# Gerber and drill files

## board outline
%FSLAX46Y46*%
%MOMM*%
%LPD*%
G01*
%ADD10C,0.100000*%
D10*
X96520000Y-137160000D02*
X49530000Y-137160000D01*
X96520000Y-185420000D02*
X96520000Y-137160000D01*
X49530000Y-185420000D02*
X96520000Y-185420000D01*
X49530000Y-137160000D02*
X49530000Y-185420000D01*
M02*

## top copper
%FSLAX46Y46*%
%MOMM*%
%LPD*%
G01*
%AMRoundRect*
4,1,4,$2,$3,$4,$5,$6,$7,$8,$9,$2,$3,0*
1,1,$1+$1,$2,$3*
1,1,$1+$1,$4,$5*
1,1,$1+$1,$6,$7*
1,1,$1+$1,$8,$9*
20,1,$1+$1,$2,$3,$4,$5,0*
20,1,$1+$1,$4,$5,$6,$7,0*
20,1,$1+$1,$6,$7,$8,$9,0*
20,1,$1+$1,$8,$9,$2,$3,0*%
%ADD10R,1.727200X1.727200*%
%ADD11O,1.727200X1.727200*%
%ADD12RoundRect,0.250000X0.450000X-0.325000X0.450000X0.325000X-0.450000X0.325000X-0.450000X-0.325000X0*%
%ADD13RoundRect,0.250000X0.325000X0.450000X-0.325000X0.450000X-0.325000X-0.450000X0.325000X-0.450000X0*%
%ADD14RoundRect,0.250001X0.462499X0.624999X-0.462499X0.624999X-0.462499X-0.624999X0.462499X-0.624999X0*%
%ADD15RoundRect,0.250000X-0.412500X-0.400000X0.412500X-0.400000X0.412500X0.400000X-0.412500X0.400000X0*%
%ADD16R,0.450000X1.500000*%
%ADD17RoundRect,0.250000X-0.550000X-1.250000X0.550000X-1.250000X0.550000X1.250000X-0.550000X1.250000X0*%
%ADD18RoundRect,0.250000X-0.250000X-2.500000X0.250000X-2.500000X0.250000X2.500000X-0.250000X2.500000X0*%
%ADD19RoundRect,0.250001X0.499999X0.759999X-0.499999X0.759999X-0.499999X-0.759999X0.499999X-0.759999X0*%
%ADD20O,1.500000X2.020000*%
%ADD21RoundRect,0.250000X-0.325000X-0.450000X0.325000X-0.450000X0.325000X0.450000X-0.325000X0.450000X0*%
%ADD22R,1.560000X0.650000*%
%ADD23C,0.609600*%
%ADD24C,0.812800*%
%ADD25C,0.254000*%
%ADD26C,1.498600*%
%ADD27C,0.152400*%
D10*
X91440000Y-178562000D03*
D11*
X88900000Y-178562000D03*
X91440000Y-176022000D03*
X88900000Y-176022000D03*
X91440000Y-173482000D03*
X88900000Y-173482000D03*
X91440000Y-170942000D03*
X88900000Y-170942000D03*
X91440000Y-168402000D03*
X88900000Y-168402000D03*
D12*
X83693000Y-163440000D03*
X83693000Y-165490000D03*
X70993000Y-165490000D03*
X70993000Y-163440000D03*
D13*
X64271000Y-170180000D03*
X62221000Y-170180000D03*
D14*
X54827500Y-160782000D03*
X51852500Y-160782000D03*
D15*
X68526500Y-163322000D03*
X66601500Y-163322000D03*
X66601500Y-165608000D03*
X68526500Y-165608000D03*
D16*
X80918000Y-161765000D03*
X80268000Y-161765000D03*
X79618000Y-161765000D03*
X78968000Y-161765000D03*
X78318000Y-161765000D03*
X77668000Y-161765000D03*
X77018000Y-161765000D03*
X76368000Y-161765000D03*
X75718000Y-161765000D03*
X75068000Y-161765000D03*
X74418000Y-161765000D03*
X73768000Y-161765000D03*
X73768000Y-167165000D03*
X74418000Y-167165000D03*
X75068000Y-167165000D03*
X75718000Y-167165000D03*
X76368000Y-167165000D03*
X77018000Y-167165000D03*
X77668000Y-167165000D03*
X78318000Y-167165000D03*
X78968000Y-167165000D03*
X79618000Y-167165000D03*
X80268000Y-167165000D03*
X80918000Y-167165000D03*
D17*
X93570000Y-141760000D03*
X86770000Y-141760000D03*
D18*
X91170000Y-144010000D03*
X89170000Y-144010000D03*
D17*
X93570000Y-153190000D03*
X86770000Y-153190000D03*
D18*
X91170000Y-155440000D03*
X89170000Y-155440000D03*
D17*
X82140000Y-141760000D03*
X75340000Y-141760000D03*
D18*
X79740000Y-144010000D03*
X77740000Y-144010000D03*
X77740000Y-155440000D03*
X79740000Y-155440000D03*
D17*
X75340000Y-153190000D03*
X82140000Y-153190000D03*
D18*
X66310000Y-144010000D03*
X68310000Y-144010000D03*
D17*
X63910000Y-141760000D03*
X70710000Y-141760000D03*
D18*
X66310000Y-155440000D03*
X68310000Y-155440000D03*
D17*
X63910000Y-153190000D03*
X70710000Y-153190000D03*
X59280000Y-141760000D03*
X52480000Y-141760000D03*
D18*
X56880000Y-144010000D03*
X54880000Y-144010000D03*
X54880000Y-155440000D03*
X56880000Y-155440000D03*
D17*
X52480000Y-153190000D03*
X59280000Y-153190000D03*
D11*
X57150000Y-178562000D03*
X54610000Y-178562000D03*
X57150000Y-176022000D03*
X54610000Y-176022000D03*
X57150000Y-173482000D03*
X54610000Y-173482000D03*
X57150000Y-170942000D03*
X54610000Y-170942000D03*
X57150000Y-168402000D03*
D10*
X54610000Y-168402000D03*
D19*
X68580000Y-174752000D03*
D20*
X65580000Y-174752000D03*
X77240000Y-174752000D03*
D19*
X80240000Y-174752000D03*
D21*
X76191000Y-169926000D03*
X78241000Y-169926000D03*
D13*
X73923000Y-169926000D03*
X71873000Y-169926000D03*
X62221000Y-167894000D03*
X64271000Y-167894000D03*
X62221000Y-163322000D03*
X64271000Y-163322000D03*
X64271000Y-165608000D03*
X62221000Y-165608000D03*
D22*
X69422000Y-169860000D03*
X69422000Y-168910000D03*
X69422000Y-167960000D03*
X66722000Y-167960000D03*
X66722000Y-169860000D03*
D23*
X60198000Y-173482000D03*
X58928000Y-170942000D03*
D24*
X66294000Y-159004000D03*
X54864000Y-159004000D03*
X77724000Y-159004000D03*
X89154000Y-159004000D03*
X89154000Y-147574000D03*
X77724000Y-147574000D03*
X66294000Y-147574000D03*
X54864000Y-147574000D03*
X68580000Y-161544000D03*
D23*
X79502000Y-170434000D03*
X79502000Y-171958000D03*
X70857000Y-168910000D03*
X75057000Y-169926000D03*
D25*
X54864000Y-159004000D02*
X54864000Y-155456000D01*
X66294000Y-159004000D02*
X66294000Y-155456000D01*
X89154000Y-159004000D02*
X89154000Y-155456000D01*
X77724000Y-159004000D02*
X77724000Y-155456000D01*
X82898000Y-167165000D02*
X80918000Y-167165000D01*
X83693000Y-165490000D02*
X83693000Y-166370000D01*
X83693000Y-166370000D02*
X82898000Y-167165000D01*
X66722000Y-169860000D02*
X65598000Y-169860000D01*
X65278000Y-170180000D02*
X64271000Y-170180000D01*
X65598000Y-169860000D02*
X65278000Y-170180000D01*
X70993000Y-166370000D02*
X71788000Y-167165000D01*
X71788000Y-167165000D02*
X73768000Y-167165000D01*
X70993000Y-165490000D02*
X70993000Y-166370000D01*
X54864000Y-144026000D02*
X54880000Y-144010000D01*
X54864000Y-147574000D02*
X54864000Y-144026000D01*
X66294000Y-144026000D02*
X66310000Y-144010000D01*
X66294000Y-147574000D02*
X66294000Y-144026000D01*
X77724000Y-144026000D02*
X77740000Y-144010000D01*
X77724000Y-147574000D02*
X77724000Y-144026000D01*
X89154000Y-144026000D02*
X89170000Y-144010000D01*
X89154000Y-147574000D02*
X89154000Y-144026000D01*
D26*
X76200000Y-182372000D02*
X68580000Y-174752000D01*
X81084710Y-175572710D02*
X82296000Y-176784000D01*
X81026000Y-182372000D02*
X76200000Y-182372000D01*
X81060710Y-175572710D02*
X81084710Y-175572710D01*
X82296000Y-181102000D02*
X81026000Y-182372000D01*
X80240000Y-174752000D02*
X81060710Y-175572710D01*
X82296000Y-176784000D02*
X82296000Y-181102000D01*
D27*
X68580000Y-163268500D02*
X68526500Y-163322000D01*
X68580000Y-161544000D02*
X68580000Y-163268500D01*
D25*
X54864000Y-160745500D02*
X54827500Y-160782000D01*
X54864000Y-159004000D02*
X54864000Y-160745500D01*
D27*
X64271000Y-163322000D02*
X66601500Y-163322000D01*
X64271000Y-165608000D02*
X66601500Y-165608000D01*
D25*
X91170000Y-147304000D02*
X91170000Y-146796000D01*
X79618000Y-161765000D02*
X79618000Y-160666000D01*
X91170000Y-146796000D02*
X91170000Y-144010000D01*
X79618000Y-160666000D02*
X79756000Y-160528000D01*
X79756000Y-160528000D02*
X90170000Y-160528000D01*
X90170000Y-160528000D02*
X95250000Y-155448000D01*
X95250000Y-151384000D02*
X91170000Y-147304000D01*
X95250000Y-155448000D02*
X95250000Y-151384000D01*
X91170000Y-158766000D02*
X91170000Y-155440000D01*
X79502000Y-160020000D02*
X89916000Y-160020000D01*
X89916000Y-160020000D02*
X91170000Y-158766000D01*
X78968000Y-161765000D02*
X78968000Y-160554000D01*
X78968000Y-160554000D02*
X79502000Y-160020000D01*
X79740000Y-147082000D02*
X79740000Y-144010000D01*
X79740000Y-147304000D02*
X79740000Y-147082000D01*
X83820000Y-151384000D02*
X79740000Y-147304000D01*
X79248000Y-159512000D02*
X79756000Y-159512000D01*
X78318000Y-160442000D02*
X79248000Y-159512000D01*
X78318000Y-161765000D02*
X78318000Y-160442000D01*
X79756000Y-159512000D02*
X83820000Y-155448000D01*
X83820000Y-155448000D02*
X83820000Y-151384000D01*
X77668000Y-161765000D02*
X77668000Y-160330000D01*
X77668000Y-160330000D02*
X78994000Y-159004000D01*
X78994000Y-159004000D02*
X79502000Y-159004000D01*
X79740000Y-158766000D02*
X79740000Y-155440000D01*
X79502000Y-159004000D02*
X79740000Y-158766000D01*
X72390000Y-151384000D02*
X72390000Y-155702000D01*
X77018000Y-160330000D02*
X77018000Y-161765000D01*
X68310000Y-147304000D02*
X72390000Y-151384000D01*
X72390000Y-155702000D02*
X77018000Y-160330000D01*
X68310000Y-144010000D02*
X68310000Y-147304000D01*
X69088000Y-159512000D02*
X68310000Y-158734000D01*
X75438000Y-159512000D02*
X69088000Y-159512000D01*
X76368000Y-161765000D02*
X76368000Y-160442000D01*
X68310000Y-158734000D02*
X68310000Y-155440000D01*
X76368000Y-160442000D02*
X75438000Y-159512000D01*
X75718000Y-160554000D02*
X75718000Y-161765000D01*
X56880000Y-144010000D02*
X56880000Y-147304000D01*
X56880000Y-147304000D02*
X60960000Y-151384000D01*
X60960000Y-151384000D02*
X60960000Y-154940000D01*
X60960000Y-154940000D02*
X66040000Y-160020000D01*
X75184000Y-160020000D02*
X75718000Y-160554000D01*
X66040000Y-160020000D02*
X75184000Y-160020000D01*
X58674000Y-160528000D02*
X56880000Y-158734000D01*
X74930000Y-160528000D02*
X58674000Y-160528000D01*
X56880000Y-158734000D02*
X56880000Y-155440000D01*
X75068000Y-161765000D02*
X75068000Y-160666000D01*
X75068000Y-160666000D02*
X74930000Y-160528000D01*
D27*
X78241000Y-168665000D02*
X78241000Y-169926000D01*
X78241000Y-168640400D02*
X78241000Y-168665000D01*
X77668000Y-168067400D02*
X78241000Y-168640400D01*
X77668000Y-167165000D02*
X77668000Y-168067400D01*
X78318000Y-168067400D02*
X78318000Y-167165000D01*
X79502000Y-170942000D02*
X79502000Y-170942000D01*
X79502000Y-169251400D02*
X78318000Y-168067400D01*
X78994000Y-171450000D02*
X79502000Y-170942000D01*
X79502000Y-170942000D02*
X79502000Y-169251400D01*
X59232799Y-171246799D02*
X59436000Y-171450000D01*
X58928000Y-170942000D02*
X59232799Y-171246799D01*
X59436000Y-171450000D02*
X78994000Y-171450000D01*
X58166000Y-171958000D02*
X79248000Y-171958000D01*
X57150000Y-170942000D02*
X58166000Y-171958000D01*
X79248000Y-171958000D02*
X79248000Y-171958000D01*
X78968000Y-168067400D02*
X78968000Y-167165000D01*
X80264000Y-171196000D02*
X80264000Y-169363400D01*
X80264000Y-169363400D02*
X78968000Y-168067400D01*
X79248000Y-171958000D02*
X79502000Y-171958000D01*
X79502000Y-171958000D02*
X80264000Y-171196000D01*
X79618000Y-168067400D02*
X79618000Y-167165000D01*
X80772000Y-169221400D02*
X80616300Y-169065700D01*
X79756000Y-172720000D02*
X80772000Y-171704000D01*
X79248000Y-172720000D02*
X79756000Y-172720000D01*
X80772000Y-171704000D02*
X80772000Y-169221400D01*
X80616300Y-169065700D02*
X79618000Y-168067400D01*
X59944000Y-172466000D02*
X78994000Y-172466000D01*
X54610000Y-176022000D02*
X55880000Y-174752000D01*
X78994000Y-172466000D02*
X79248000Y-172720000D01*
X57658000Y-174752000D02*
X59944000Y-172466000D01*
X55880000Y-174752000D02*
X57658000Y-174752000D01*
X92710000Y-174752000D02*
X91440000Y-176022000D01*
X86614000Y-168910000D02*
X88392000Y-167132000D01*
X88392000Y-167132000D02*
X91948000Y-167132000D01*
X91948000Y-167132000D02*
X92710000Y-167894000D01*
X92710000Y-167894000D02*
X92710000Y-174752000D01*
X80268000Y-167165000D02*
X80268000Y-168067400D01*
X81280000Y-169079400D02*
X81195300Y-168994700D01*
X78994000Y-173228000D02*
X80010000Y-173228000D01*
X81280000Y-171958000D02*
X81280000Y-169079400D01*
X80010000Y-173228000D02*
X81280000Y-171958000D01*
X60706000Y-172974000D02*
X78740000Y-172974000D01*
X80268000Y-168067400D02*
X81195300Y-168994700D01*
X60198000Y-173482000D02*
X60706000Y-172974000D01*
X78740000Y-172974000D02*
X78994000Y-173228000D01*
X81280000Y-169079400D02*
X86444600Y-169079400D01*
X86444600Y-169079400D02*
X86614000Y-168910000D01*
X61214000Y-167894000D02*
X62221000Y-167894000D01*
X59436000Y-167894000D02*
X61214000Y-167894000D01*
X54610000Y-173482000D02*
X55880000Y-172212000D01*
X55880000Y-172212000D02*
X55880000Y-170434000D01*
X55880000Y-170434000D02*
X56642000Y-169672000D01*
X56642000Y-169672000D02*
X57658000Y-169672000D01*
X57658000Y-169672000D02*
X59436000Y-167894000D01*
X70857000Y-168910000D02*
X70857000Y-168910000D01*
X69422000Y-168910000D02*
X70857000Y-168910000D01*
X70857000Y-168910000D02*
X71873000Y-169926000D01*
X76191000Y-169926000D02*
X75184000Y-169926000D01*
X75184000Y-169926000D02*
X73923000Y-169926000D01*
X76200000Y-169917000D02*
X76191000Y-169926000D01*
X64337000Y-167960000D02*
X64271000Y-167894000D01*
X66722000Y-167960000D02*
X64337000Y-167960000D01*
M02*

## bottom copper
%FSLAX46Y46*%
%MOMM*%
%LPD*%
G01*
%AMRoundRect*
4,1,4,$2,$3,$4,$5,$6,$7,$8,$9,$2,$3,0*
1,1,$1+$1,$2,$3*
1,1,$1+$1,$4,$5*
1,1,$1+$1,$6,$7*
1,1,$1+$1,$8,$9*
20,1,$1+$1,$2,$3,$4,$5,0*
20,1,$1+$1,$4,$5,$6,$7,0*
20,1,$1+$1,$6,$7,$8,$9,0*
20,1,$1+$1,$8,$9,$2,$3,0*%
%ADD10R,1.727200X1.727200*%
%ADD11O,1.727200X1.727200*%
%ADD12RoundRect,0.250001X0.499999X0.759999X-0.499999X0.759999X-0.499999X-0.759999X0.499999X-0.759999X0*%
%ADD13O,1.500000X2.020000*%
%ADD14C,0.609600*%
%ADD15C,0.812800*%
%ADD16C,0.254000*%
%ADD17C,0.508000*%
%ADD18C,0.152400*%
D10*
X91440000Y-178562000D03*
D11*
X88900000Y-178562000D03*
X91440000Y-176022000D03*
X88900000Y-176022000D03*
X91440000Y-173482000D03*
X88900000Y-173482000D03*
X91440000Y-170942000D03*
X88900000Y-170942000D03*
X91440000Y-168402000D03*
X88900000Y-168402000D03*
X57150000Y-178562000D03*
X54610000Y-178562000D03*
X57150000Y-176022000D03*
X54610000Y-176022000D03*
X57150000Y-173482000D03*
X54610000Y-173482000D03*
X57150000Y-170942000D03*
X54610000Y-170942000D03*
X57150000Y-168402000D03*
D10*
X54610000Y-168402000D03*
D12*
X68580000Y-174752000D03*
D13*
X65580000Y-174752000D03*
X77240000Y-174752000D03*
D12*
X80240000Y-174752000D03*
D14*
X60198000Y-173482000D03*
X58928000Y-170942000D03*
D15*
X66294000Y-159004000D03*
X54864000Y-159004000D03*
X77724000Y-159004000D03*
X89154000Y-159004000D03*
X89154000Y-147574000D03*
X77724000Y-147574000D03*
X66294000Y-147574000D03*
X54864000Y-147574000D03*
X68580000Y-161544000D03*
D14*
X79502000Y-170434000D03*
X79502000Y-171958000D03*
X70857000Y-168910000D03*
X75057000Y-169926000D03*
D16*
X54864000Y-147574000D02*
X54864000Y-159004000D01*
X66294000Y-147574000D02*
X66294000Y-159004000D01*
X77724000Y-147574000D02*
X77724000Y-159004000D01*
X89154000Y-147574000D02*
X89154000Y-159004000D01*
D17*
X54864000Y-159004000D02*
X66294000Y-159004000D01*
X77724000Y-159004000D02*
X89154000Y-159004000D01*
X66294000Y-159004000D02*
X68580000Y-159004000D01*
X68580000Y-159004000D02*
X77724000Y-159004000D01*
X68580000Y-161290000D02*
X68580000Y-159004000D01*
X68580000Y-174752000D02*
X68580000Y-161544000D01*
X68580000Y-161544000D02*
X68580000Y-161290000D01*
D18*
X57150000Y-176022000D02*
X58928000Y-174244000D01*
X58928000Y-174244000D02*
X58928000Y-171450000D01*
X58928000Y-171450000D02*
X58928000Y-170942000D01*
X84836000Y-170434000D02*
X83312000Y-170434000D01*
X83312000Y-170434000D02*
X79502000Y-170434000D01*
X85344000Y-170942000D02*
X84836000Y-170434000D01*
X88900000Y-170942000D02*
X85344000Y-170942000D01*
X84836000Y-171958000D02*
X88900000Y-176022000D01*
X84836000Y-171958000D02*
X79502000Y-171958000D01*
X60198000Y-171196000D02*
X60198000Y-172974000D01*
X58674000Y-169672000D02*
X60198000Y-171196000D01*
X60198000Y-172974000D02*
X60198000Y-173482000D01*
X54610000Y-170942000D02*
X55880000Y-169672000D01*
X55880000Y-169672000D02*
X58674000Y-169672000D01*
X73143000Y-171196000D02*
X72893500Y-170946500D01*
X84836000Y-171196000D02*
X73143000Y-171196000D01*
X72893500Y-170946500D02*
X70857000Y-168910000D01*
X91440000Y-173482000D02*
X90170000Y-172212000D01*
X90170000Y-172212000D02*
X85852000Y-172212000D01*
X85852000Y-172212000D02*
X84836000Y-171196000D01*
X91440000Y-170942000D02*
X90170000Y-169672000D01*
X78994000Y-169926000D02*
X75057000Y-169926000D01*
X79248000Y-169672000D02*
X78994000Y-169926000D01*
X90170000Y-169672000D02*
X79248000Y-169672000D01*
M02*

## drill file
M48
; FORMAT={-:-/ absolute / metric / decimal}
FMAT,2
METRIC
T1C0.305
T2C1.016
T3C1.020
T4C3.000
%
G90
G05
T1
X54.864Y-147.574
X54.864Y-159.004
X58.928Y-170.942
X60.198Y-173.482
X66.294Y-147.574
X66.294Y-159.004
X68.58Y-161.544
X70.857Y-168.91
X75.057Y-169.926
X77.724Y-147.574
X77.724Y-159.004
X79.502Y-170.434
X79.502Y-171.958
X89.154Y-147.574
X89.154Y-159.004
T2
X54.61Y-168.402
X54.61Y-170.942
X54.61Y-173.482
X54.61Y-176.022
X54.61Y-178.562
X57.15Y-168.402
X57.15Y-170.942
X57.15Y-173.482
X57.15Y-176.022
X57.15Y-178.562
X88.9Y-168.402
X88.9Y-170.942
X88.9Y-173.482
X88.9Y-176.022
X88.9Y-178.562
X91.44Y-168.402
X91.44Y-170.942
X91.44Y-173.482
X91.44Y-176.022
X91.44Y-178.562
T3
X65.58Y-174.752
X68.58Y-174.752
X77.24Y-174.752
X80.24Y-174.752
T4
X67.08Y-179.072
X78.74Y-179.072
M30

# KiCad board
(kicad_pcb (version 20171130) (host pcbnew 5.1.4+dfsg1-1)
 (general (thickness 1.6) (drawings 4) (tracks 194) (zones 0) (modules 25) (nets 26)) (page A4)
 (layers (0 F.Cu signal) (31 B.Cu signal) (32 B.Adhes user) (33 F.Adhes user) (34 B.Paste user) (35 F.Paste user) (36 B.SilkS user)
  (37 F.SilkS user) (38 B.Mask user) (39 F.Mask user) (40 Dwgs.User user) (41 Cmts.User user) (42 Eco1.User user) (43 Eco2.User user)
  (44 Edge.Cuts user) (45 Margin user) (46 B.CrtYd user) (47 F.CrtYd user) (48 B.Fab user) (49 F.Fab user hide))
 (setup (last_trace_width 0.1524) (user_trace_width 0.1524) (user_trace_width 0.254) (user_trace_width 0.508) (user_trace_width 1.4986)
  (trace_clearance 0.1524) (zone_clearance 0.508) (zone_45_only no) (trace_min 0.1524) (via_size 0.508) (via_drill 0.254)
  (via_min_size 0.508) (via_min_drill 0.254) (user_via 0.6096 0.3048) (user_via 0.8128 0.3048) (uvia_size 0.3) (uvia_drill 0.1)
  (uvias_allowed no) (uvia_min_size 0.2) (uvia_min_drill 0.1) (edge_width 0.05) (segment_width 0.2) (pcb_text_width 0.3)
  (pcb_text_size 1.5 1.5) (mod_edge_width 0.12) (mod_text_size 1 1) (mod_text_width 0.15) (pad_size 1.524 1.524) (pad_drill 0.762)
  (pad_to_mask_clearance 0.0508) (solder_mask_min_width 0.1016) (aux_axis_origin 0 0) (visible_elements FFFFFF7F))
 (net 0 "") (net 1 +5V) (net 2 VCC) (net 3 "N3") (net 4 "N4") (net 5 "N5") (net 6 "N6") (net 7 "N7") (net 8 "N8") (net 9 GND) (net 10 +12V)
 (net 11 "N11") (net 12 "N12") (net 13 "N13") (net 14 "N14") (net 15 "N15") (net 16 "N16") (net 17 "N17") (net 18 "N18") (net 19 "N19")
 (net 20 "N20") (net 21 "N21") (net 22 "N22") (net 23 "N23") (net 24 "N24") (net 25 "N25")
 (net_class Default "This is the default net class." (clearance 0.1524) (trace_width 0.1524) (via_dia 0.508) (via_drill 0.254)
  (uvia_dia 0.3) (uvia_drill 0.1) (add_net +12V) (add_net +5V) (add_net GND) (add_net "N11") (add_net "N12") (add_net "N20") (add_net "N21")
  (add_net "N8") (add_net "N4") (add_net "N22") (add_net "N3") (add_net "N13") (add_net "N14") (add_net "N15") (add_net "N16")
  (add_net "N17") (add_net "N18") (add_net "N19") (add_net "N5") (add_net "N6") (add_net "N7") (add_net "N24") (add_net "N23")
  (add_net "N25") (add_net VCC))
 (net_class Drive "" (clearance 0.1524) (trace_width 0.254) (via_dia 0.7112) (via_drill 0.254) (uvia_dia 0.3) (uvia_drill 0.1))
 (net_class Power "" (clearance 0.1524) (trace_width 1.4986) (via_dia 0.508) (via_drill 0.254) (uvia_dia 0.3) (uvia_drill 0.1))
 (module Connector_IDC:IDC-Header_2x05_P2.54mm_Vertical (layer F.Cu) (at 91.44 178.562 180)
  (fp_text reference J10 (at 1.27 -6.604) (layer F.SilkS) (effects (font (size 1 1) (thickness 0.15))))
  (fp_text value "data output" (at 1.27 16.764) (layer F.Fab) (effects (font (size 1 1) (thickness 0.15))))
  (pad 1 thru_hole rect (at 0 0 180) (size 1.7272 1.7272) (drill 1.016) (layers *.Cu *.Mask) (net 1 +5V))
  (pad 2 thru_hole oval (at 2.54 0 180) (size 1.7272 1.7272) (drill 1.016) (layers *.Cu *.Mask) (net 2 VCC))
  (pad 3 thru_hole oval (at 0 2.54 180) (size 1.7272 1.7272) (drill 1.016) (layers *.Cu *.Mask) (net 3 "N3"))
  (pad 4 thru_hole oval (at 2.54 2.54 180) (size 1.7272 1.7272) (drill 1.016) (layers *.Cu *.Mask) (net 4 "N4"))
  (pad 5 thru_hole oval (at 0 5.08 180) (size 1.7272 1.7272) (drill 1.016) (layers *.Cu *.Mask) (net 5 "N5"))
  (pad 6 thru_hole oval (at 2.54 5.08 180) (size 1.7272 1.7272) (drill 1.016) (layers *.Cu *.Mask) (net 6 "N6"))
  (pad 7 thru_hole oval (at 0 7.62 180) (size 1.7272 1.7272) (drill 1.016) (layers *.Cu *.Mask) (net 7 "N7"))
  (pad 8 thru_hole oval (at 2.54 7.62 180) (size 1.7272 1.7272) (drill 1.016) (layers *.Cu *.Mask) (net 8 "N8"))
  (pad 9 thru_hole oval (at 0 10.16 180) (size 1.7272 1.7272) (drill 1.016) (layers *.Cu *.Mask) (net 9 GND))
  (pad 10 thru_hole oval (at 2.54 10.16 180) (size 1.7272 1.7272) (drill 1.016) (layers *.Cu *.Mask) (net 9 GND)))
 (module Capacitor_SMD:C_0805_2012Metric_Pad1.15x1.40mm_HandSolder (layer F.Cu) (at 83.693 164.465 90)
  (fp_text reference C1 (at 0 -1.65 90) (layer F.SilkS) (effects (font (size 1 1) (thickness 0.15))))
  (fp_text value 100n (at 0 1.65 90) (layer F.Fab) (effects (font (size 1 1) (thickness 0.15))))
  (pad 2 smd roundrect (at 1.025 0 90) (size 1.15 1.4) (layers F.Cu F.Paste F.Mask) (roundrect_rratio 0.217391) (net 9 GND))
  (pad 1 smd roundrect (at -1.025 0 90) (size 1.15 1.4) (layers F.Cu F.Paste F.Mask) (roundrect_rratio 0.217391) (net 1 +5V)))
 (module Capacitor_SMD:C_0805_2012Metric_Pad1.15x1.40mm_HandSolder (layer F.Cu) (at 70.993 164.465 90)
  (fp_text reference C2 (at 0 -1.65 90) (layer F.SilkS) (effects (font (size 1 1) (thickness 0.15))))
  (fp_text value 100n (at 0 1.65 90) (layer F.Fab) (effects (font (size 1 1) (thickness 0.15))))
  (pad 1 smd roundrect (at -1.025 0 90) (size 1.15 1.4) (layers F.Cu F.Paste F.Mask) (roundrect_rratio 0.217391) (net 2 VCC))
  (pad 2 smd roundrect (at 1.025 0 90) (size 1.15 1.4) (layers F.Cu F.Paste F.Mask) (roundrect_rratio 0.217391) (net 9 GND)))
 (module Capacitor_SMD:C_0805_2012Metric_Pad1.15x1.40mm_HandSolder (layer F.Cu) (at 63.246 170.18 180)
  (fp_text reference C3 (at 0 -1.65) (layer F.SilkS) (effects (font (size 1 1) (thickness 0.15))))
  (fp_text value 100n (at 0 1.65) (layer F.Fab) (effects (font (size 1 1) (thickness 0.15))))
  (pad 1 smd roundrect (at -1.025 0 180) (size 1.15 1.4) (layers F.Cu F.Paste F.Mask) (roundrect_rratio 0.217391) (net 2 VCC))
  (pad 2 smd roundrect (at 1.025 0 180) (size 1.15 1.4) (layers F.Cu F.Paste F.Mask) (roundrect_rratio 0.217391) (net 9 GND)))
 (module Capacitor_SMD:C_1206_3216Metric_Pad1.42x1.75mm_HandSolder (layer F.Cu) (at 53.34 160.782 180)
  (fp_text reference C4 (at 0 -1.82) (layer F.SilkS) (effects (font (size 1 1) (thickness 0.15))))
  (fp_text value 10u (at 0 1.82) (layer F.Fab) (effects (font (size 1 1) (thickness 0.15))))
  (pad 1 smd roundrect (at -1.4875 0 180) (size 1.425 1.75) (layers F.Cu F.Paste F.Mask) (roundrect_rratio 0.175439) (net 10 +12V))
  (pad 2 smd roundrect (at 1.4875 0 180) (size 1.425 1.75) (layers F.Cu F.Paste F.Mask) (roundrect_rratio 0.175439) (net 9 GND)))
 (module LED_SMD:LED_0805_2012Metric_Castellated (layer F.Cu) (at 67.564 163.322)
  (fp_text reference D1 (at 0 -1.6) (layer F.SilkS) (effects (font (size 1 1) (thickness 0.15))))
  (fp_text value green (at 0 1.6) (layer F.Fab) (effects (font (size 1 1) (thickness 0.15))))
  (pad 2 smd roundrect (at 0.9625 0) (size 1.325 1.3) (layers F.Cu F.Paste F.Mask) (roundrect_rratio 0.192308) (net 10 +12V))
  (pad 1 smd roundrect (at -0.9625 0) (size 1.325 1.3) (layers F.Cu F.Paste F.Mask) (roundrect_rratio 0.192308) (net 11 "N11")))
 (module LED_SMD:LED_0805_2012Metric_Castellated (layer F.Cu) (at 67.564 165.608)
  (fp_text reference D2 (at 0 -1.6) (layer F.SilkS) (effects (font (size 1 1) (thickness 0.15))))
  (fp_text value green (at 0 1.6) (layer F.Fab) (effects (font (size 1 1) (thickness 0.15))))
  (pad 1 smd roundrect (at -0.9625 0) (size 1.325 1.3) (layers F.Cu F.Paste F.Mask) (roundrect_rratio 0.192308) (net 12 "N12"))
  (pad 2 smd roundrect (at 0.9625 0) (size 1.325 1.3) (layers F.Cu F.Paste F.Mask) (roundrect_rratio 0.192308) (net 1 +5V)))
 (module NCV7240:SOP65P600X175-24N (layer F.Cu) (at 77.343 164.465 270)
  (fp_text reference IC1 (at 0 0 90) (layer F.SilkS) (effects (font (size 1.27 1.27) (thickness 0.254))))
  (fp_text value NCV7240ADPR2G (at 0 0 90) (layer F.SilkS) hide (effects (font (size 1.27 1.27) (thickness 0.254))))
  (pad 1 smd rect (at -2.7 -3.575) (size 0.45 1.5) (layers F.Cu F.Paste F.Mask) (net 9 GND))
  (pad 2 smd rect (at -2.7 -2.925) (size 0.45 1.5) (layers F.Cu F.Paste F.Mask) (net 9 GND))
  (pad 3 smd rect (at -2.7 -2.275) (size 0.45 1.5) (layers F.Cu F.Paste F.Mask) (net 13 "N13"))
  (pad 4 smd rect (at -2.7 -1.625) (size 0.45 1.5) (layers F.Cu F.Paste F.Mask) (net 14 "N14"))
  (pad 5 smd rect (at -2.7 -0.975) (size 0.45 1.5) (layers F.Cu F.Paste F.Mask) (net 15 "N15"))
  (pad 6 smd rect (at -2.7 -0.325) (size 0.45 1.5) (layers F.Cu F.Paste F.Mask) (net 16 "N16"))
  (pad 7 smd rect (at -2.7 0.325) (size 0.45 1.5) (layers F.Cu F.Paste F.Mask) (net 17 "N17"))
  (pad 8 smd rect (at -2.7 0.975) (size 0.45 1.5) (layers F.Cu F.Paste F.Mask) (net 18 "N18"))
  (pad 9 smd rect (at -2.7 1.625) (size 0.45 1.5) (layers F.Cu F.Paste F.Mask) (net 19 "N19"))
  (pad 10 smd rect (at -2.7 2.275) (size 0.45 1.5) (layers F.Cu F.Paste F.Mask) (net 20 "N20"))
  (pad 11 smd rect (at -2.7 2.925) (size 0.45 1.5) (layers F.Cu F.Paste F.Mask) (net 9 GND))
  (pad 12 smd rect (at -2.7 3.575) (size 0.45 1.5) (layers F.Cu F.Paste F.Mask) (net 9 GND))
  (pad 13 smd rect (at 2.7 3.575) (size 0.45 1.5) (layers F.Cu F.Paste F.Mask) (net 2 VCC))
  (pad 14 smd rect (at 2.7 2.925) (size 0.45 1.5) (layers F.Cu F.Paste F.Mask) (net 9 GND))
  (pad 15 smd rect (at 2.7 2.275) (size 0.45 1.5) (layers F.Cu F.Paste F.Mask) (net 9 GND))
  (pad 16 smd rect (at 2.7 1.625) (size 0.45 1.5) (layers F.Cu F.Paste F.Mask) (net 9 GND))
  (pad 17 smd rect (at 2.7 0.975) (size 0.45 1.5) (layers F.Cu F.Paste F.Mask) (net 9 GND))
  (pad 18 smd rect (at 2.7 0.325) (size 0.45 1.5) (layers F.Cu F.Paste F.Mask) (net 9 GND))
  (pad 19 smd rect (at 2.7 -0.325) (size 0.45 1.5) (layers F.Cu F.Paste F.Mask) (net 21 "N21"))
  (pad 20 smd rect (at 2.7 -0.975) (size 0.45 1.5) (layers F.Cu F.Paste F.Mask) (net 8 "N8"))
  (pad 21 smd rect (at 2.7 -1.625) (size 0.45 1.5) (layers F.Cu F.Paste F.Mask) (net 4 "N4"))
  (pad 22 smd rect (at 2.7 -2.275) (size 0.45 1.5) (layers F.Cu F.Paste F.Mask) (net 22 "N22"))
  (pad 23 smd rect (at 2.7 -2.925) (size 0.45 1.5) (layers F.Cu F.Paste F.Mask) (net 3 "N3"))
  (pad 24 smd rect (at 2.7 -3.575) (size 0.45 1.5) (layers F.Cu F.Paste F.Mask) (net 1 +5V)))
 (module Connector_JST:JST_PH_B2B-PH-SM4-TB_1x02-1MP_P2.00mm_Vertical (layer F.Cu) (at 90.17 143.51)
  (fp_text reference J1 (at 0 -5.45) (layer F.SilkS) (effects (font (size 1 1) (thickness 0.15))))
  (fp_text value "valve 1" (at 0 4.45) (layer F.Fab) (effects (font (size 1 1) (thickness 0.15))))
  (pad MP smd roundrect (at 3.4 -1.75) (size 1.6 3) (layers F.Cu F.Paste F.Mask) (roundrect_rratio 0.15625))
  (pad MP smd roundrect (at -3.4 -1.75) (size 1.6 3) (layers F.Cu F.Paste F.Mask) (roundrect_rratio 0.15625))
  (pad 2 smd roundrect (at 1 0.5) (size 1 5.5) (layers F.Cu F.Paste F.Mask) (roundrect_rratio 0.25) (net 13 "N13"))
  (pad 1 smd roundrect (at -1 0.5) (size 1 5.5) (layers F.Cu F.Paste F.Mask) (roundrect_rratio 0.25) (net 10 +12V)))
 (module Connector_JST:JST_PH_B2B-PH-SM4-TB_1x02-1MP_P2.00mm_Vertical (layer F.Cu) (at 90.17 154.94)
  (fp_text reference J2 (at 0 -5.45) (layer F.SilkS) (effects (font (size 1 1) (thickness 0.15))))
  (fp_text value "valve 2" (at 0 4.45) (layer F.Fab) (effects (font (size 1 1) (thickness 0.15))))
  (pad MP smd roundrect (at 3.4 -1.75) (size 1.6 3) (layers F.Cu F.Paste F.Mask) (roundrect_rratio 0.15625))
  (pad MP smd roundrect (at -3.4 -1.75) (size 1.6 3) (layers F.Cu F.Paste F.Mask) (roundrect_rratio 0.15625))
  (pad 2 smd roundrect (at 1 0.5) (size 1 5.5) (layers F.Cu F.Paste F.Mask) (roundrect_rratio 0.25) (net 14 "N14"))
  (pad 1 smd roundrect (at -1 0.5) (size 1 5.5) (layers F.Cu F.Paste F.Mask) (roundrect_rratio 0.25) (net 10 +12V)))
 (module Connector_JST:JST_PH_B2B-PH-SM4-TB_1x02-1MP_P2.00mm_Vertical (layer F.Cu) (at 78.74 143.51)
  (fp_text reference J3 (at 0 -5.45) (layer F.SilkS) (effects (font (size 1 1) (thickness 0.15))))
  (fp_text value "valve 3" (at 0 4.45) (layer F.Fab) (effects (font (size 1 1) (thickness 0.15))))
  (pad MP smd roundrect (at 3.4 -1.75) (size 1.6 3) (layers F.Cu F.Paste F.Mask) (roundrect_rratio 0.15625))
  (pad MP smd roundrect (at -3.4 -1.75) (size 1.6 3) (layers F.Cu F.Paste F.Mask) (roundrect_rratio 0.15625))
  (pad 2 smd roundrect (at 1 0.5) (size 1 5.5) (layers F.Cu F.Paste F.Mask) (roundrect_rratio 0.25) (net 15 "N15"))
  (pad 1 smd roundrect (at -1 0.5) (size 1 5.5) (layers F.Cu F.Paste F.Mask) (roundrect_rratio 0.25) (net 10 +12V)))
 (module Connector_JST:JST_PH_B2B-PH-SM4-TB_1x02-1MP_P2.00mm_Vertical (layer F.Cu) (at 78.74 154.94)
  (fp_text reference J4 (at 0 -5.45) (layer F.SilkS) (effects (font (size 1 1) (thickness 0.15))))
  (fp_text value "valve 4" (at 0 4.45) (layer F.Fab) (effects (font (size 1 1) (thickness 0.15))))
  (pad 1 smd roundrect (at -1 0.5) (size 1 5.5) (layers F.Cu F.Paste F.Mask) (roundrect_rratio 0.25) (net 10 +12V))
  (pad 2 smd roundrect (at 1 0.5) (size 1 5.5) (layers F.Cu F.Paste F.Mask) (roundrect_rratio 0.25) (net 16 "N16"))
  (pad MP smd roundrect (at -3.4 -1.75) (size 1.6 3) (layers F.Cu F.Paste F.Mask) (roundrect_rratio 0.15625))
  (pad MP smd roundrect (at 3.4 -1.75) (size 1.6 3) (layers F.Cu F.Paste F.Mask) (roundrect_rratio 0.15625)))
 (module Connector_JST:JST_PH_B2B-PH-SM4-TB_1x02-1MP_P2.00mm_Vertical (layer F.Cu) (at 67.31 143.51)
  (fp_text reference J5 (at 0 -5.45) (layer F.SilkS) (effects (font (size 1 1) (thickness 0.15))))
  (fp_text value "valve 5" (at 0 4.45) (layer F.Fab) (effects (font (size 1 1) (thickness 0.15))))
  (pad 1 smd roundrect (at -1 0.5) (size 1 5.5) (layers F.Cu F.Paste F.Mask) (roundrect_rratio 0.25) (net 10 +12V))
  (pad 2 smd roundrect (at 1 0.5) (size 1 5.5) (layers F.Cu F.Paste F.Mask) (roundrect_rratio 0.25) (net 17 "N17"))
  (pad MP smd roundrect (at -3.4 -1.75) (size 1.6 3) (layers F.Cu F.Paste F.Mask) (roundrect_rratio 0.15625))
  (pad MP smd roundrect (at 3.4 -1.75) (size 1.6 3) (layers F.Cu F.Paste F.Mask) (roundrect_rratio 0.15625)))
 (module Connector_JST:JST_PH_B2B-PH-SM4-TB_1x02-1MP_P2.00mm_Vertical (layer F.Cu) (at 67.31 154.94)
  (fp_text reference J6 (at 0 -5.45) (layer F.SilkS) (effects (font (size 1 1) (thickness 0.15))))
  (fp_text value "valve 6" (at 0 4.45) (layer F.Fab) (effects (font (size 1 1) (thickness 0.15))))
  (pad 1 smd roundrect (at -1 0.5) (size 1 5.5) (layers F.Cu F.Paste F.Mask) (roundrect_rratio 0.25) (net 10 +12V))
  (pad 2 smd roundrect (at 1 0.5) (size 1 5.5) (layers F.Cu F.Paste F.Mask) (roundrect_rratio 0.25) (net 18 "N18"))
  (pad MP smd roundrect (at -3.4 -1.75) (size 1.6 3) (layers F.Cu F.Paste F.Mask) (roundrect_rratio 0.15625))
  (pad MP smd roundrect (at 3.4 -1.75) (size 1.6 3) (layers F.Cu F.Paste F.Mask) (roundrect_rratio 0.15625)))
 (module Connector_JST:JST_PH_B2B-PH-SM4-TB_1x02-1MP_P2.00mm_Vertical (layer F.Cu) (at 55.88 143.51)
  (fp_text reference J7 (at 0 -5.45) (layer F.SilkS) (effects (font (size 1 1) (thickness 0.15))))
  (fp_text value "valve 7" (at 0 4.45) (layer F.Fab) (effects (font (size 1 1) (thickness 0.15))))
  (pad MP smd roundrect (at 3.4 -1.75) (size 1.6 3) (layers F.Cu F.Paste F.Mask) (roundrect_rratio 0.15625))
  (pad MP smd roundrect (at -3.4 -1.75) (size 1.6 3) (layers F.Cu F.Paste F.Mask) (roundrect_rratio 0.15625))
  (pad 2 smd roundrect (at 1 0.5) (size 1 5.5) (layers F.Cu F.Paste F.Mask) (roundrect_rratio 0.25) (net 19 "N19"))
  (pad 1 smd roundrect (at -1 0.5) (size 1 5.5) (layers F.Cu F.Paste F.Mask) (roundrect_rratio 0.25) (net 10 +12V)))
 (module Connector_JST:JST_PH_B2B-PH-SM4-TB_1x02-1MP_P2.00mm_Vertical (layer F.Cu) (at 55.88 154.94)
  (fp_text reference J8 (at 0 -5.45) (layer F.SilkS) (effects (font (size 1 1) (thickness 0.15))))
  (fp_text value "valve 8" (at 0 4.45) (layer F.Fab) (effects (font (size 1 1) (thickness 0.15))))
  (pad 1 smd roundrect (at -1 0.5) (size 1 5.5) (layers F.Cu F.Paste F.Mask) (roundrect_rratio 0.25) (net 10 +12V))
  (pad 2 smd roundrect (at 1 0.5) (size 1 5.5) (layers F.Cu F.Paste F.Mask) (roundrect_rratio 0.25) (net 20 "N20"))
  (pad MP smd roundrect (at -3.4 -1.75) (size 1.6 3) (layers F.Cu F.Paste F.Mask) (roundrect_rratio 0.15625))
  (pad MP smd roundrect (at 3.4 -1.75) (size 1.6 3) (layers F.Cu F.Paste F.Mask) (roundrect_rratio 0.15625)))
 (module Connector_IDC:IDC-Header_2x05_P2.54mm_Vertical (layer F.Cu) (at 54.61 168.402)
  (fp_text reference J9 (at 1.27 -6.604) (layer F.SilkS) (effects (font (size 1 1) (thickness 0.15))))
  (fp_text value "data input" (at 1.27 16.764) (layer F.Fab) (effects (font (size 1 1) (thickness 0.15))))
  (pad 10 thru_hole oval (at 2.54 10.16) (size 1.7272 1.7272) (drill 1.016) (layers *.Cu *.Mask) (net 9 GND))
  (pad 9 thru_hole oval (at 0 10.16) (size 1.7272 1.7272) (drill 1.016) (layers *.Cu *.Mask) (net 9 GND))
  (pad 8 thru_hole oval (at 2.54 7.62) (size 1.7272 1.7272) (drill 1.016) (layers *.Cu *.Mask) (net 8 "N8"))
  (pad 7 thru_hole oval (at 0 7.62) (size 1.7272 1.7272) (drill 1.016) (layers *.Cu *.Mask) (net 22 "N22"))
  (pad 6 thru_hole oval (at 2.54 5.08) (size 1.7272 1.7272) (drill 1.016) (layers *.Cu *.Mask) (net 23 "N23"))
  (pad 5 thru_hole oval (at 0 5.08) (size 1.7272 1.7272) (drill 1.016) (layers *.Cu *.Mask) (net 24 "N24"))
  (pad 4 thru_hole oval (at 2.54 2.54) (size 1.7272 1.7272) (drill 1.016) (layers *.Cu *.Mask) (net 4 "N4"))
  (pad 3 thru_hole oval (at 0 2.54) (size 1.7272 1.7272) (drill 1.016) (layers *.Cu *.Mask) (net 3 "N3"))
  (pad 2 thru_hole oval (at 2.54 0) (size 1.7272 1.7272) (drill 1.016) (layers *.Cu *.Mask) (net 2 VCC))
  (pad 1 thru_hole rect (at 0 0) (size 1.7272 1.7272) (drill 1.016) (layers *.Cu *.Mask) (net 1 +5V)))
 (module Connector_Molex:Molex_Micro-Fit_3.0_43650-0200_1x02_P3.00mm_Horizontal (layer F.Cu) (at 68.58 174.752 180)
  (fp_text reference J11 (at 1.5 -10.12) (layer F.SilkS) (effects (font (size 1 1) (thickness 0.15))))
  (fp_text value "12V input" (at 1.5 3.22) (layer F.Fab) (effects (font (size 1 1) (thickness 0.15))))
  (pad "" np_thru_hole circle (at 1.5 -4.32 180) (size 3 3) (drill 3) (layers *.Cu *.Mask))
  (pad 1 thru_hole roundrect (at 0 0 180) (size 1.5 2.02) (drill 1.02) (layers *.Cu *.Mask) (roundrect_rratio 0.166667) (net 10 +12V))
  (pad 2 thru_hole oval (at 3 0 180) (size 1.5 2.02) (drill 1.02) (layers *.Cu *.Mask) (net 9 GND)))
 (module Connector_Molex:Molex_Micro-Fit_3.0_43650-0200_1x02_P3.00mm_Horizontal (layer F.Cu) (at 80.24 174.752 180)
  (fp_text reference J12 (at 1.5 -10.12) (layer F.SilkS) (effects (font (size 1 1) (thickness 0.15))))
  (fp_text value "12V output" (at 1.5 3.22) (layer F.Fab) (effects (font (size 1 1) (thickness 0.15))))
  (pad 2 thru_hole oval (at 3 0 180) (size 1.5 2.02) (drill 1.02) (layers *.Cu *.Mask) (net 9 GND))
  (pad 1 thru_hole roundrect (at 0 0 180) (size 1.5 2.02) (drill 1.02) (layers *.Cu *.Mask) (roundrect_rratio 0.166667) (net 10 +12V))
  (pad "" np_thru_hole circle (at 1.5 -4.32 180) (size 3 3) (drill 3) (layers *.Cu *.Mask)))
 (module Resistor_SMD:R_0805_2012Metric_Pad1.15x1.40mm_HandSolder (layer F.Cu) (at 77.216 169.926)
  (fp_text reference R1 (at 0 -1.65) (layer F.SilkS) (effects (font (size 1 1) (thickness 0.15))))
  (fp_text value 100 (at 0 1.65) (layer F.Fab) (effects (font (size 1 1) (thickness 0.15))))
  (pad 1 smd roundrect (at -1.025 0) (size 1.15 1.4) (layers F.Cu F.Paste F.Mask) (roundrect_rratio 0.217391) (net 7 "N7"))
  (pad 2 smd roundrect (at 1.025 0) (size 1.15 1.4) (layers F.Cu F.Paste F.Mask) (roundrect_rratio 0.217391) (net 21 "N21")))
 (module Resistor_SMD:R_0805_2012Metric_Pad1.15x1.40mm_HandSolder (layer F.Cu) (at 72.898 169.926 180)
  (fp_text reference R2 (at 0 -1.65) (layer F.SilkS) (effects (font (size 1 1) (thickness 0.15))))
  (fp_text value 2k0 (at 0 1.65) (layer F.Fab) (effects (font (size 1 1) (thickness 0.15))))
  (pad 1 smd roundrect (at -1.025 0 180) (size 1.15 1.4) (layers F.Cu F.Paste F.Mask) (roundrect_rratio 0.217391) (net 7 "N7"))
  (pad 2 smd roundrect (at 1.025 0 180) (size 1.15 1.4) (layers F.Cu F.Paste F.Mask) (roundrect_rratio 0.217391) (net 5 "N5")))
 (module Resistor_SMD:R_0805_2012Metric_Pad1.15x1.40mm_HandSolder (layer F.Cu) (at 63.246 167.894 180)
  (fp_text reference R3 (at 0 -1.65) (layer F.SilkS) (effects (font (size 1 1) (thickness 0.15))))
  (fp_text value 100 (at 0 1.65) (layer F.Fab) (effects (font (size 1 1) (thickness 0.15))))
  (pad 2 smd roundrect (at 1.025 0 180) (size 1.15 1.4) (layers F.Cu F.Paste F.Mask) (roundrect_rratio 0.217391) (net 24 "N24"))
  (pad 1 smd roundrect (at -1.025 0 180) (size 1.15 1.4) (layers F.Cu F.Paste F.Mask) (roundrect_rratio 0.217391) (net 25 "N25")))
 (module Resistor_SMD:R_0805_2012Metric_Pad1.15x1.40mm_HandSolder (layer F.Cu) (at 63.246 163.322 180)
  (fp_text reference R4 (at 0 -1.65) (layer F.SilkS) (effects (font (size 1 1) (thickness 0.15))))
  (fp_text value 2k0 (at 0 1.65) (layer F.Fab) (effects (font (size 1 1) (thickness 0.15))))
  (pad 2 smd roundrect (at 1.025 0 180) (size 1.15 1.4) (layers F.Cu F.Paste F.Mask) (roundrect_rratio 0.217391) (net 9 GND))
  (pad 1 smd roundrect (at -1.025 0 180) (size 1.15 1.4) (layers F.Cu F.Paste F.Mask) (roundrect_rratio 0.217391) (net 11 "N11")))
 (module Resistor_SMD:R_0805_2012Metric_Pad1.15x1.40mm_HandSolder (layer F.Cu) (at 63.246 165.608 180)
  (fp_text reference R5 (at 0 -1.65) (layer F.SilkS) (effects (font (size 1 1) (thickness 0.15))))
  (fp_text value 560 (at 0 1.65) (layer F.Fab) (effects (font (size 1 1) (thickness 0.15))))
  (pad 1 smd roundrect (at -1.025 0 180) (size 1.15 1.4) (layers F.Cu F.Paste F.Mask) (roundrect_rratio 0.217391) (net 12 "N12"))
  (pad 2 smd roundrect (at 1.025 0 180) (size 1.15 1.4) (layers F.Cu F.Paste F.Mask) (roundrect_rratio 0.217391) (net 9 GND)))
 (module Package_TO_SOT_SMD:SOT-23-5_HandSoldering (layer F.Cu) (at 68.072 168.91 180)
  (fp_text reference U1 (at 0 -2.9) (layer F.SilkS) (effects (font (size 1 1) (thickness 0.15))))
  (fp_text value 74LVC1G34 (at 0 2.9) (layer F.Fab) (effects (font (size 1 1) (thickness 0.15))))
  (pad 1 smd rect (at -1.35 -0.95 180) (size 1.56 0.65) (layers F.Cu F.Paste F.Mask))
  (pad 2 smd rect (at -1.35 0 180) (size 1.56 0.65) (layers F.Cu F.Paste F.Mask) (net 5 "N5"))
  (pad 3 smd rect (at -1.35 0.95 180) (size 1.56 0.65) (layers F.Cu F.Paste F.Mask) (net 9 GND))
  (pad 4 smd rect (at 1.35 0.95 180) (size 1.56 0.65) (layers F.Cu F.Paste F.Mask) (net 25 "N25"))
  (pad 5 smd rect (at 1.35 -0.95 180) (size 1.56 0.65) (layers F.Cu F.Paste F.Mask) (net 2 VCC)))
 (gr_line (start 96.52 137.16) (end 49.53 137.16) (layer Edge.Cuts) (width 0.1))
 (gr_line (start 96.52 185.42) (end 96.52 137.16) (layer Edge.Cuts) (width 0.1))
 (gr_line (start 49.53 185.42) (end 96.52 185.42) (layer Edge.Cuts) (width 0.1))
 (gr_line (start 49.53 137.16) (end 49.53 185.42) (layer Edge.Cuts) (width 0.1))
 (via (at 60.198 173.482) (size 0.6096) (drill 0.3048) (layers F.Cu B.Cu) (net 3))
 (via (at 58.928 170.942) (size 0.6096) (drill 0.3048) (layers F.Cu B.Cu) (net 8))
 (segment (start 54.864 159.004) (end 54.864 155.456) (width 0.254) (layer F.Cu) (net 10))
 (via (at 66.294 159.004) (size 0.8128) (drill 0.3048) (layers F.Cu B.Cu) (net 10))
 (via (at 54.864 159.004) (size 0.8128) (drill 0.3048) (layers F.Cu B.Cu) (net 10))
 (segment (start 66.294 159.004) (end 66.294 155.456) (width 0.254) (layer F.Cu) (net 10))
 (via (at 77.724 159.004) (size 0.8128) (drill 0.3048) (layers F.Cu B.Cu) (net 10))
 (segment (start 89.154 159.004) (end 89.154 155.456) (width 0.254) (layer F.Cu) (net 10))
 (segment (start 77.724 159.004) (end 77.724 155.456) (width 0.254) (layer F.Cu) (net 10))
 (via (at 89.154 159.004) (size 0.8128) (drill 0.3048) (layers F.Cu B.Cu) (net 10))
 (via (at 89.154 147.574) (size 0.8128) (drill 0.3048) (layers F.Cu B.Cu) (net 10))
 (via (at 77.724 147.574) (size 0.8128) (drill 0.3048) (layers F.Cu B.Cu) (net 10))
 (via (at 66.294 147.574) (size 0.8128) (drill 0.3048) (layers F.Cu B.Cu) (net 10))
 (via (at 54.864 147.574) (size 0.8128) (drill 0.3048) (layers F.Cu B.Cu) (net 10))
 (segment (start 82.898 167.165) (end 80.918 167.165) (width 0.254) (layer F.Cu) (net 1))
 (segment (start 83.693 165.49) (end 83.693 166.37) (width 0.254) (layer F.Cu) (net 1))
 (segment (start 83.693 166.37) (end 82.898 167.165) (width 0.254) (layer F.Cu) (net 1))
 (segment (start 66.722 169.86) (end 65.598 169.86) (width 0.254) (layer F.Cu) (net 2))
 (segment (start 65.278 170.18) (end 64.271 170.18) (width 0.254) (layer F.Cu) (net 2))
 (segment (start 65.598 169.86) (end 65.278 170.18) (width 0.254) (layer F.Cu) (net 2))
 (segment (start 70.993 166.37) (end 71.788 167.165) (width 0.254) (layer F.Cu) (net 2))
 (segment (start 71.788 167.165) (end 73.768 167.165) (width 0.254) (layer F.Cu) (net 2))
 (segment (start 70.993 165.49) (end 70.993 166.37) (width 0.254) (layer F.Cu) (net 2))
 (segment (start 54.864 144.026) (end 54.88 144.01) (width 0.254) (layer F.Cu) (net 10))
 (segment (start 54.864 147.574) (end 54.864 144.026) (width 0.254) (layer F.Cu) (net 10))
 (segment (start 66.294 144.026) (end 66.31 144.01) (width 0.254) (layer F.Cu) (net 10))
 (segment (start 66.294 147.574) (end 66.294 144.026) (width 0.254) (layer F.Cu) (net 10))
 (segment (start 77.724 144.026) (end 77.74 144.01) (width 0.254) (layer F.Cu) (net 10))
 (segment (start 77.724 147.574) (end 77.724 144.026) (width 0.254) (layer F.Cu) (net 10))
 (segment (start 89.154 144.026) (end 89.17 144.01) (width 0.254) (layer F.Cu) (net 10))
 (segment (start 89.154 147.574) (end 89.154 144.026) (width 0.254) (layer F.Cu) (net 10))
 (segment (start 54.864 147.574) (end 54.864 159.004) (width 0.254) (layer B.Cu) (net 10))
 (segment (start 66.294 147.574) (end 66.294 159.004) (width 0.254) (layer B.Cu) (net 10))
 (segment (start 77.724 147.574) (end 77.724 159.004) (width 0.254) (layer B.Cu) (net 10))
 (segment (start 89.154 147.574) (end 89.154 159.004) (width 0.254) (layer B.Cu) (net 10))
 (segment (start 54.864 159.004) (end 66.294 159.004) (width 0.508) (layer B.Cu) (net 10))
 (segment (start 77.724 159.004) (end 89.154 159.004) (width 0.508) (layer B.Cu) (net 10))
 (segment (start 76.2 182.372) (end 68.58 174.752) (width 1.4986) (layer F.Cu) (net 10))
 (segment (start 81.08471 175.57271) (end 82.296 176.784) (width 1.4986) (layer F.Cu) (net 10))
 (segment (start 81.026 182.372) (end 76.2 182.372) (width 1.4986) (layer F.Cu) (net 10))
 (segment (start 81.06071 175.57271) (end 81.08471 175.57271) (width 1.4986) (layer F.Cu) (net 10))
 (segment (start 82.296 181.102) (end 81.026 182.372) (width 1.4986) (layer F.Cu) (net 10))
 (segment (start 80.24 174.752) (end 81.06071 175.57271) (width 1.4986) (layer F.Cu) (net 10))
 (segment (start 82.296 176.784) (end 82.296 181.102) (width 1.4986) (layer F.Cu) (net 10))
 (segment (start 68.58 163.2685) (end 68.5265 163.322) (width 0.1524) (layer F.Cu) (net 10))
 (segment (start 68.58 161.544) (end 68.58 163.2685) (width 0.1524) (layer F.Cu) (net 10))
 (segment (start 66.294 159.004) (end 68.58 159.004) (width 0.508) (layer B.Cu) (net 10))
 (segment (start 68.58 159.004) (end 77.724 159.004) (width 0.508) (layer B.Cu) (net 10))
 (segment (start 54.864 160.7455) (end 54.8275 160.782) (width 0.254) (layer F.Cu) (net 10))
 (segment (start 54.864 159.004) (end 54.864 160.7455) (width 0.254) (layer F.Cu) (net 10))
 (segment (start 68.58 161.29) (end 68.58 159.004) (width 0.508) (layer B.Cu) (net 10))
 (segment (start 68.58 174.752) (end 68.58 161.544) (width 0.508) (layer B.Cu) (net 10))
 (segment (start 68.58 161.544) (end 68.58 161.29) (width 0.508) (layer B.Cu) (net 10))
 (via (at 68.58 161.544) (size 0.8128) (drill 0.3048) (layers F.Cu B.Cu) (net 10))
 (segment (start 64.271 163.322) (end 66.6015 163.322) (width 0.1524) (layer F.Cu) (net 11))
 (segment (start 64.271 165.608) (end 66.6015 165.608) (width 0.1524) (layer F.Cu) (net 12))
 (segment (start 91.17 147.304) (end 91.17 146.796) (width 0.254) (layer F.Cu) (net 13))
 (segment (start 79.618 161.765) (end 79.618 160.666) (width 0.254) (layer F.Cu) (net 13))
 (segment (start 91.17 146.796) (end 91.17 144.01) (width 0.254) (layer F.Cu) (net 13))
 (segment (start 79.618 160.666) (end 79.756 160.528) (width 0.254) (layer F.Cu) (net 13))
 (segment (start 79.756 160.528) (end 90.17 160.528) (width 0.254) (layer F.Cu) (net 13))
 (segment (start 90.17 160.528) (end 95.25 155.448) (width 0.254) (layer F.Cu) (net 13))
 (segment (start 95.25 151.384) (end 91.17 147.304) (width 0.254) (layer F.Cu) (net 13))
 (segment (start 95.25 155.448) (end 95.25 151.384) (width 0.254) (layer F.Cu) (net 13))
 (segment (start 91.17 158.766) (end 91.17 155.44) (width 0.254) (layer F.Cu) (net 14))
 (segment (start 79.502 160.02) (end 89.916 160.02) (width 0.254) (layer F.Cu) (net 14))
 (segment (start 89.916 160.02) (end 91.17 158.766) (width 0.254) (layer F.Cu) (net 14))
 (segment (start 78.968 161.765) (end 78.968 160.554) (width 0.254) (layer F.Cu) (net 14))
 (segment (start 78.968 160.554) (end 79.502 160.02) (width 0.254) (layer F.Cu) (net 14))
 (segment (start 79.74 147.082) (end 79.74 144.01) (width 0.254) (layer F.Cu) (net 15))
 (segment (start 79.74 147.304) (end 79.74 147.082) (width 0.254) (layer F.Cu) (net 15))
 (segment (start 83.82 151.384) (end 79.74 147.304) (width 0.254) (layer F.Cu) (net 15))
 (segment (start 79.248 159.512) (end 79.756 159.512) (width 0.254) (layer F.Cu) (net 15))
 (segment (start 78.318 160.442) (end 79.248 159.512) (width 0.254) (layer F.Cu) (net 15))
 (segment (start 78.318 161.765) (end 78.318 160.442) (width 0.254) (layer F.Cu) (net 15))
 (segment (start 79.756 159.512) (end 83.82 155.448) (width 0.254) (layer F.Cu) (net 15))
 (segment (start 83.82 155.448) (end 83.82 151.384) (width 0.254) (layer F.Cu) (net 15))
 (segment (start 77.668 161.765) (end 77.668 160.33) (width 0.254) (layer F.Cu) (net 16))
 (segment (start 77.668 160.33) (end 78.994 159.004) (width 0.254) (layer F.Cu) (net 16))
 (segment (start 78.994 159.004) (end 79.502 159.004) (width 0.254) (layer F.Cu) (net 16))
 (segment (start 79.74 158.766) (end 79.74 155.44) (width 0.254) (layer F.Cu) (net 16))
 (segment (start 79.502 159.004) (end 79.74 158.766) (width 0.254) (layer F.Cu) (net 16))
 (segment (start 72.39 151.384) (end 72.39 155.702) (width 0.254) (layer F.Cu) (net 17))
 (segment (start 77.018 160.33) (end 77.018 161.765) (width 0.254) (layer F.Cu) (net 17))
 (segment (start 68.31 147.304) (end 72.39 151.384) (width 0.254) (layer F.Cu) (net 17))
 (segment (start 72.39 155.702) (end 77.018 160.33) (width 0.254) (layer F.Cu) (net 17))
 (segment (start 68.31 144.01) (end 68.31 147.304) (width 0.254) (layer F.Cu) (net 17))
 (segment (start 69.088 159.512) (end 68.31 158.734) (width 0.254) (layer F.Cu) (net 18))
 (segment (start 75.438 159.512) (end 69.088 159.512) (width 0.254) (layer F.Cu) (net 18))
 (segment (start 76.368 161.765) (end 76.368 160.442) (width 0.254) (layer F.Cu) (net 18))
 (segment (start 68.31 158.734) (end 68.31 155.44) (width 0.254) (layer F.Cu) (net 18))
 (segment (start 76.368 160.442) (end 75.438 159.512) (width 0.254) (layer F.Cu) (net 18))
 (segment (start 75.718 160.554) (end 75.718 161.765) (width 0.254) (layer F.Cu) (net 19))
 (segment (start 56.88 144.01) (end 56.88 147.304) (width 0.254) (layer F.Cu) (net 19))
 (segment (start 56.88 147.304) (end 60.96 151.384) (width 0.254) (layer F.Cu) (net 19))
 (segment (start 60.96 151.384) (end 60.96 154.94) (width 0.254) (layer F.Cu) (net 19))
 (segment (start 60.96 154.94) (end 66.04 160.02) (width 0.254) (layer F.Cu) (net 19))
 (segment (start 75.184 160.02) (end 75.718 160.554) (width 0.254) (layer F.Cu) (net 19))
 (segment (start 66.04 160.02) (end 75.184 160.02) (width 0.254) (layer F.Cu) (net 19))
 (segment (start 58.674 160.528) (end 56.88 158.734) (width 0.254) (layer F.Cu) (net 20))
 (segment (start 74.93 160.528) (end 58.674 160.528) (width 0.254) (layer F.Cu) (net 20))
 (segment (start 56.88 158.734) (end 56.88 155.44) (width 0.254) (layer F.Cu) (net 20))
 (segment (start 75.068 161.765) (end 75.068 160.666) (width 0.254) (layer F.Cu) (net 20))
 (segment (start 75.068 160.666) (end 74.93 160.528) (width 0.254) (layer F.Cu) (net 20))
 (segment (start 78.241 168.665) (end 78.241 169.926) (width 0.1524) (layer F.Cu) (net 21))
 (segment (start 78.241 168.6404) (end 78.241 168.665) (width 0.1524) (layer F.Cu) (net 21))
 (segment (start 77.668 168.0674) (end 78.241 168.6404) (width 0.1524) (layer F.Cu) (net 21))
 (segment (start 77.668 167.165) (end 77.668 168.0674) (width 0.1524) (layer F.Cu) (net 21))
 (segment (start 57.15 176.022) (end 58.928 174.244) (width 0.1524) (layer B.Cu) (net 8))
 (segment (start 58.928 174.244) (end 58.928 171.45) (width 0.1524) (layer B.Cu) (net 8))
 (segment (start 78.318 168.0674) (end 78.318 167.165) (width 0.1524) (layer F.Cu) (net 8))
 (segment (start 79.502 170.942) (end 79.502 170.942) (width 0.1524) (layer F.Cu) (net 8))
 (segment (start 79.502 169.2514) (end 78.318 168.0674) (width 0.1524) (layer F.Cu) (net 8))
 (segment (start 78.994 171.45) (end 79.502 170.942) (width 0.1524) (layer F.Cu) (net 8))
 (segment (start 79.502 170.942) (end 79.502 169.2514) (width 0.1524) (layer F.Cu) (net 8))
 (via (at 79.502 170.434) (size 0.6096) (drill 0.3048) (layers F.Cu B.Cu) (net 8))
 (segment (start 59.232799 171.246799) (end 59.436 171.45) (width 0.1524) (layer F.Cu) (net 8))
 (segment (start 58.928 170.942) (end 59.232799 171.246799) (width 0.1524) (layer F.Cu) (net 8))
 (segment (start 59.436 171.45) (end 78.994 171.45) (width 0.1524) (layer F.Cu) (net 8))
 (segment (start 58.928 171.45) (end 58.928 170.942) (width 0.1524) (layer B.Cu) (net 8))
 (segment (start 84.836 170.434) (end 83.312 170.434) (width 0.1524) (layer B.Cu) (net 8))
 (segment (start 83.312 170.434) (end 79.502 170.434) (width 0.1524) (layer B.Cu) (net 8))
 (segment (start 85.344 170.942) (end 84.836 170.434) (width 0.1524) (layer B.Cu) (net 8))
 (segment (start 88.9 170.942) (end 85.344 170.942) (width 0.1524) (layer B.Cu) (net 8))
 (segment (start 58.166 171.958) (end 79.248 171.958) (width 0.1524) (layer F.Cu) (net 4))
 (segment (start 57.15 170.942) (end 58.166 171.958) (width 0.1524) (layer F.Cu) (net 4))
 (segment (start 79.248 171.958) (end 79.248 171.958) (width 0.1524) (layer F.Cu) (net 4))
 (via (at 79.502 171.958) (size 0.6096) (drill 0.3048) (layers F.Cu B.Cu) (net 4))
 (segment (start 84.836 171.958) (end 88.9 176.022) (width 0.1524) (layer B.Cu) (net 4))
 (segment (start 78.968 168.0674) (end 78.968 167.165) (width 0.1524) (layer F.Cu) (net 4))
 (segment (start 80.264 171.196) (end 80.264 169.3634) (width 0.1524) (layer F.Cu) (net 4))
 (segment (start 80.264 169.3634) (end 78.968 168.0674) (width 0.1524) (layer F.Cu) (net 4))
 (segment (start 79.248 171.958) (end 79.502 171.958) (width 0.1524) (layer F.Cu) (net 4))
 (segment (start 79.502 171.958) (end 80.264 171.196) (width 0.1524) (layer F.Cu) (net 4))
 (segment (start 84.836 171.958) (end 79.502 171.958) (width 0.1524) (layer B.Cu) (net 4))
 (segment (start 79.618 168.0674) (end 79.618 167.165) (width 0.1524) (layer F.Cu) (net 22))
 (segment (start 80.772 169.2214) (end 80.6163 169.0657) (width 0.1524) (layer F.Cu) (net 22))
 (segment (start 79.756 172.72) (end 80.772 171.704) (width 0.1524) (layer F.Cu) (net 22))
 (segment (start 79.248 172.72) (end 79.756 172.72) (width 0.1524) (layer F.Cu) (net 22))
 (segment (start 80.772 171.704) (end 80.772 169.2214) (width 0.1524) (layer F.Cu) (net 22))
 (segment (start 80.6163 169.0657) (end 79.618 168.0674) (width 0.1524) (layer F.Cu) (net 22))
 (segment (start 59.944 172.466) (end 78.994 172.466) (width 0.1524) (layer F.Cu) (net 22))
 (segment (start 54.61 176.022) (end 55.88 174.752) (width 0.1524) (layer F.Cu) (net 22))
 (segment (start 78.994 172.466) (end 79.248 172.72) (width 0.1524) (layer F.Cu) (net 22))
 (segment (start 57.658 174.752) (end 59.944 172.466) (width 0.1524) (layer F.Cu) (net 22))
 (segment (start 55.88 174.752) (end 57.658 174.752) (width 0.1524) (layer F.Cu) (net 22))
 (segment (start 92.71 174.752) (end 91.44 176.022) (width 0.1524) (layer F.Cu) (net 3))
 (segment (start 86.614 168.91) (end 88.392 167.132) (width 0.1524) (layer F.Cu) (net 3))
 (segment (start 88.392 167.132) (end 91.948 167.132) (width 0.1524) (layer F.Cu) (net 3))
 (segment (start 91.948 167.132) (end 92.71 167.894) (width 0.1524) (layer F.Cu) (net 3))
 (segment (start 92.71 167.894) (end 92.71 174.752) (width 0.1524) (layer F.Cu) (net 3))
 (segment (start 60.198 171.196) (end 60.198 172.974) (width 0.1524) (layer B.Cu) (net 3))
 (segment (start 58.674 169.672) (end 60.198 171.196) (width 0.1524) (layer B.Cu) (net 3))
 (segment (start 60.198 172.974) (end 60.198 173.482) (width 0.1524) (layer B.Cu) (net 3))
 (segment (start 54.61 170.942) (end 55.88 169.672) (width 0.1524) (layer B.Cu) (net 3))
 (segment (start 55.88 169.672) (end 58.674 169.672) (width 0.1524) (layer B.Cu) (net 3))
 (segment (start 80.268 167.165) (end 80.268 168.0674) (width 0.1524) (layer F.Cu) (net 3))
 (segment (start 81.28 169.0794) (end 81.1953 168.9947) (width 0.1524) (layer F.Cu) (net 3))
 (segment (start 78.994 173.228) (end 80.01 173.228) (width 0.1524) (layer F.Cu) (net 3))
 (segment (start 81.28 171.958) (end 81.28 169.0794) (width 0.1524) (layer F.Cu) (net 3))
 (segment (start 80.01 173.228) (end 81.28 171.958) (width 0.1524) (layer F.Cu) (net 3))
 (segment (start 60.706 172.974) (end 78.74 172.974) (width 0.1524) (layer F.Cu) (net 3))
 (segment (start 80.268 168.0674) (end 81.1953 168.9947) (width 0.1524) (layer F.Cu) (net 3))
 (segment (start 60.198 173.482) (end 60.706 172.974) (width 0.1524) (layer F.Cu) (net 3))
 (segment (start 78.74 172.974) (end 78.994 173.228) (width 0.1524) (layer F.Cu) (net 3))
 (segment (start 81.28 169.0794) (end 86.4446 169.0794) (width 0.1524) (layer F.Cu) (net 3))
 (segment (start 86.4446 169.0794) (end 86.614 168.91) (width 0.1524) (layer F.Cu) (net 3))
 (segment (start 61.214 167.894) (end 62.221 167.894) (width 0.1524) (layer F.Cu) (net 24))
 (segment (start 59.436 167.894) (end 61.214 167.894) (width 0.1524) (layer F.Cu) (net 24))
 (segment (start 54.61 173.482) (end 55.88 172.212) (width 0.1524) (layer F.Cu) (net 24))
 (segment (start 55.88 172.212) (end 55.88 170.434) (width 0.1524) (layer F.Cu) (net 24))
 (segment (start 55.88 170.434) (end 56.642 169.672) (width 0.1524) (layer F.Cu) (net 24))
 (segment (start 56.642 169.672) (end 57.658 169.672) (width 0.1524) (layer F.Cu) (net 24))
 (segment (start 57.658 169.672) (end 59.436 167.894) (width 0.1524) (layer F.Cu) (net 24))
 (segment (start 70.857 168.91) (end 70.857 168.91) (width 0.1524) (layer F.Cu) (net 5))
 (segment (start 69.422 168.91) (end 70.857 168.91) (width 0.1524) (layer F.Cu) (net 5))
 (segment (start 70.857 168.91) (end 71.873 169.926) (width 0.1524) (layer F.Cu) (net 5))
 (via (at 70.857 168.91) (size 0.6096) (drill 0.3048) (layers F.Cu B.Cu) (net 5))
 (segment (start 73.143 171.196) (end 72.8935 170.9465) (width 0.1524) (layer B.Cu) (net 5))
 (segment (start 84.836 171.196) (end 73.143 171.196) (width 0.1524) (layer B.Cu) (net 5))
 (segment (start 72.8935 170.9465) (end 70.857 168.91) (width 0.1524) (layer B.Cu) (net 5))
 (segment (start 91.44 173.482) (end 90.17 172.212) (width 0.1524) (layer B.Cu) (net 5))
 (segment (start 90.17 172.212) (end 85.852 172.212) (width 0.1524) (layer B.Cu) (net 5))
 (segment (start 85.852 172.212) (end 84.836 171.196) (width 0.1524) (layer B.Cu) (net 5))
 (segment (start 76.191 169.926) (end 75.184 169.926) (width 0.1524) (layer F.Cu) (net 7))
 (segment (start 75.184 169.926) (end 73.923 169.926) (width 0.1524) (layer F.Cu) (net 7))
 (via (at 75.057 169.926) (size 0.6096) (drill 0.3048) (layers F.Cu B.Cu) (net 7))
 (segment (start 76.2 169.917) (end 76.191 169.926) (width 0.1524) (layer F.Cu) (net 7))
 (segment (start 91.44 170.942) (end 90.17 169.672) (width 0.1524) (layer B.Cu) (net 7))
 (segment (start 78.994 169.926) (end 75.057 169.926) (width 0.1524) (layer B.Cu) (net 7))
 (segment (start 79.248 169.672) (end 78.994 169.926) (width 0.1524) (layer B.Cu) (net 7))
 (segment (start 90.17 169.672) (end 79.248 169.672) (width 0.1524) (layer B.Cu) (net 7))
 (segment (start 64.337 167.96) (end 64.271 167.894) (width 0.1524) (layer F.Cu) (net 25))
 (segment (start 66.722 167.96) (end 64.337 167.96) (width 0.1524) (layer F.Cu) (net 25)))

